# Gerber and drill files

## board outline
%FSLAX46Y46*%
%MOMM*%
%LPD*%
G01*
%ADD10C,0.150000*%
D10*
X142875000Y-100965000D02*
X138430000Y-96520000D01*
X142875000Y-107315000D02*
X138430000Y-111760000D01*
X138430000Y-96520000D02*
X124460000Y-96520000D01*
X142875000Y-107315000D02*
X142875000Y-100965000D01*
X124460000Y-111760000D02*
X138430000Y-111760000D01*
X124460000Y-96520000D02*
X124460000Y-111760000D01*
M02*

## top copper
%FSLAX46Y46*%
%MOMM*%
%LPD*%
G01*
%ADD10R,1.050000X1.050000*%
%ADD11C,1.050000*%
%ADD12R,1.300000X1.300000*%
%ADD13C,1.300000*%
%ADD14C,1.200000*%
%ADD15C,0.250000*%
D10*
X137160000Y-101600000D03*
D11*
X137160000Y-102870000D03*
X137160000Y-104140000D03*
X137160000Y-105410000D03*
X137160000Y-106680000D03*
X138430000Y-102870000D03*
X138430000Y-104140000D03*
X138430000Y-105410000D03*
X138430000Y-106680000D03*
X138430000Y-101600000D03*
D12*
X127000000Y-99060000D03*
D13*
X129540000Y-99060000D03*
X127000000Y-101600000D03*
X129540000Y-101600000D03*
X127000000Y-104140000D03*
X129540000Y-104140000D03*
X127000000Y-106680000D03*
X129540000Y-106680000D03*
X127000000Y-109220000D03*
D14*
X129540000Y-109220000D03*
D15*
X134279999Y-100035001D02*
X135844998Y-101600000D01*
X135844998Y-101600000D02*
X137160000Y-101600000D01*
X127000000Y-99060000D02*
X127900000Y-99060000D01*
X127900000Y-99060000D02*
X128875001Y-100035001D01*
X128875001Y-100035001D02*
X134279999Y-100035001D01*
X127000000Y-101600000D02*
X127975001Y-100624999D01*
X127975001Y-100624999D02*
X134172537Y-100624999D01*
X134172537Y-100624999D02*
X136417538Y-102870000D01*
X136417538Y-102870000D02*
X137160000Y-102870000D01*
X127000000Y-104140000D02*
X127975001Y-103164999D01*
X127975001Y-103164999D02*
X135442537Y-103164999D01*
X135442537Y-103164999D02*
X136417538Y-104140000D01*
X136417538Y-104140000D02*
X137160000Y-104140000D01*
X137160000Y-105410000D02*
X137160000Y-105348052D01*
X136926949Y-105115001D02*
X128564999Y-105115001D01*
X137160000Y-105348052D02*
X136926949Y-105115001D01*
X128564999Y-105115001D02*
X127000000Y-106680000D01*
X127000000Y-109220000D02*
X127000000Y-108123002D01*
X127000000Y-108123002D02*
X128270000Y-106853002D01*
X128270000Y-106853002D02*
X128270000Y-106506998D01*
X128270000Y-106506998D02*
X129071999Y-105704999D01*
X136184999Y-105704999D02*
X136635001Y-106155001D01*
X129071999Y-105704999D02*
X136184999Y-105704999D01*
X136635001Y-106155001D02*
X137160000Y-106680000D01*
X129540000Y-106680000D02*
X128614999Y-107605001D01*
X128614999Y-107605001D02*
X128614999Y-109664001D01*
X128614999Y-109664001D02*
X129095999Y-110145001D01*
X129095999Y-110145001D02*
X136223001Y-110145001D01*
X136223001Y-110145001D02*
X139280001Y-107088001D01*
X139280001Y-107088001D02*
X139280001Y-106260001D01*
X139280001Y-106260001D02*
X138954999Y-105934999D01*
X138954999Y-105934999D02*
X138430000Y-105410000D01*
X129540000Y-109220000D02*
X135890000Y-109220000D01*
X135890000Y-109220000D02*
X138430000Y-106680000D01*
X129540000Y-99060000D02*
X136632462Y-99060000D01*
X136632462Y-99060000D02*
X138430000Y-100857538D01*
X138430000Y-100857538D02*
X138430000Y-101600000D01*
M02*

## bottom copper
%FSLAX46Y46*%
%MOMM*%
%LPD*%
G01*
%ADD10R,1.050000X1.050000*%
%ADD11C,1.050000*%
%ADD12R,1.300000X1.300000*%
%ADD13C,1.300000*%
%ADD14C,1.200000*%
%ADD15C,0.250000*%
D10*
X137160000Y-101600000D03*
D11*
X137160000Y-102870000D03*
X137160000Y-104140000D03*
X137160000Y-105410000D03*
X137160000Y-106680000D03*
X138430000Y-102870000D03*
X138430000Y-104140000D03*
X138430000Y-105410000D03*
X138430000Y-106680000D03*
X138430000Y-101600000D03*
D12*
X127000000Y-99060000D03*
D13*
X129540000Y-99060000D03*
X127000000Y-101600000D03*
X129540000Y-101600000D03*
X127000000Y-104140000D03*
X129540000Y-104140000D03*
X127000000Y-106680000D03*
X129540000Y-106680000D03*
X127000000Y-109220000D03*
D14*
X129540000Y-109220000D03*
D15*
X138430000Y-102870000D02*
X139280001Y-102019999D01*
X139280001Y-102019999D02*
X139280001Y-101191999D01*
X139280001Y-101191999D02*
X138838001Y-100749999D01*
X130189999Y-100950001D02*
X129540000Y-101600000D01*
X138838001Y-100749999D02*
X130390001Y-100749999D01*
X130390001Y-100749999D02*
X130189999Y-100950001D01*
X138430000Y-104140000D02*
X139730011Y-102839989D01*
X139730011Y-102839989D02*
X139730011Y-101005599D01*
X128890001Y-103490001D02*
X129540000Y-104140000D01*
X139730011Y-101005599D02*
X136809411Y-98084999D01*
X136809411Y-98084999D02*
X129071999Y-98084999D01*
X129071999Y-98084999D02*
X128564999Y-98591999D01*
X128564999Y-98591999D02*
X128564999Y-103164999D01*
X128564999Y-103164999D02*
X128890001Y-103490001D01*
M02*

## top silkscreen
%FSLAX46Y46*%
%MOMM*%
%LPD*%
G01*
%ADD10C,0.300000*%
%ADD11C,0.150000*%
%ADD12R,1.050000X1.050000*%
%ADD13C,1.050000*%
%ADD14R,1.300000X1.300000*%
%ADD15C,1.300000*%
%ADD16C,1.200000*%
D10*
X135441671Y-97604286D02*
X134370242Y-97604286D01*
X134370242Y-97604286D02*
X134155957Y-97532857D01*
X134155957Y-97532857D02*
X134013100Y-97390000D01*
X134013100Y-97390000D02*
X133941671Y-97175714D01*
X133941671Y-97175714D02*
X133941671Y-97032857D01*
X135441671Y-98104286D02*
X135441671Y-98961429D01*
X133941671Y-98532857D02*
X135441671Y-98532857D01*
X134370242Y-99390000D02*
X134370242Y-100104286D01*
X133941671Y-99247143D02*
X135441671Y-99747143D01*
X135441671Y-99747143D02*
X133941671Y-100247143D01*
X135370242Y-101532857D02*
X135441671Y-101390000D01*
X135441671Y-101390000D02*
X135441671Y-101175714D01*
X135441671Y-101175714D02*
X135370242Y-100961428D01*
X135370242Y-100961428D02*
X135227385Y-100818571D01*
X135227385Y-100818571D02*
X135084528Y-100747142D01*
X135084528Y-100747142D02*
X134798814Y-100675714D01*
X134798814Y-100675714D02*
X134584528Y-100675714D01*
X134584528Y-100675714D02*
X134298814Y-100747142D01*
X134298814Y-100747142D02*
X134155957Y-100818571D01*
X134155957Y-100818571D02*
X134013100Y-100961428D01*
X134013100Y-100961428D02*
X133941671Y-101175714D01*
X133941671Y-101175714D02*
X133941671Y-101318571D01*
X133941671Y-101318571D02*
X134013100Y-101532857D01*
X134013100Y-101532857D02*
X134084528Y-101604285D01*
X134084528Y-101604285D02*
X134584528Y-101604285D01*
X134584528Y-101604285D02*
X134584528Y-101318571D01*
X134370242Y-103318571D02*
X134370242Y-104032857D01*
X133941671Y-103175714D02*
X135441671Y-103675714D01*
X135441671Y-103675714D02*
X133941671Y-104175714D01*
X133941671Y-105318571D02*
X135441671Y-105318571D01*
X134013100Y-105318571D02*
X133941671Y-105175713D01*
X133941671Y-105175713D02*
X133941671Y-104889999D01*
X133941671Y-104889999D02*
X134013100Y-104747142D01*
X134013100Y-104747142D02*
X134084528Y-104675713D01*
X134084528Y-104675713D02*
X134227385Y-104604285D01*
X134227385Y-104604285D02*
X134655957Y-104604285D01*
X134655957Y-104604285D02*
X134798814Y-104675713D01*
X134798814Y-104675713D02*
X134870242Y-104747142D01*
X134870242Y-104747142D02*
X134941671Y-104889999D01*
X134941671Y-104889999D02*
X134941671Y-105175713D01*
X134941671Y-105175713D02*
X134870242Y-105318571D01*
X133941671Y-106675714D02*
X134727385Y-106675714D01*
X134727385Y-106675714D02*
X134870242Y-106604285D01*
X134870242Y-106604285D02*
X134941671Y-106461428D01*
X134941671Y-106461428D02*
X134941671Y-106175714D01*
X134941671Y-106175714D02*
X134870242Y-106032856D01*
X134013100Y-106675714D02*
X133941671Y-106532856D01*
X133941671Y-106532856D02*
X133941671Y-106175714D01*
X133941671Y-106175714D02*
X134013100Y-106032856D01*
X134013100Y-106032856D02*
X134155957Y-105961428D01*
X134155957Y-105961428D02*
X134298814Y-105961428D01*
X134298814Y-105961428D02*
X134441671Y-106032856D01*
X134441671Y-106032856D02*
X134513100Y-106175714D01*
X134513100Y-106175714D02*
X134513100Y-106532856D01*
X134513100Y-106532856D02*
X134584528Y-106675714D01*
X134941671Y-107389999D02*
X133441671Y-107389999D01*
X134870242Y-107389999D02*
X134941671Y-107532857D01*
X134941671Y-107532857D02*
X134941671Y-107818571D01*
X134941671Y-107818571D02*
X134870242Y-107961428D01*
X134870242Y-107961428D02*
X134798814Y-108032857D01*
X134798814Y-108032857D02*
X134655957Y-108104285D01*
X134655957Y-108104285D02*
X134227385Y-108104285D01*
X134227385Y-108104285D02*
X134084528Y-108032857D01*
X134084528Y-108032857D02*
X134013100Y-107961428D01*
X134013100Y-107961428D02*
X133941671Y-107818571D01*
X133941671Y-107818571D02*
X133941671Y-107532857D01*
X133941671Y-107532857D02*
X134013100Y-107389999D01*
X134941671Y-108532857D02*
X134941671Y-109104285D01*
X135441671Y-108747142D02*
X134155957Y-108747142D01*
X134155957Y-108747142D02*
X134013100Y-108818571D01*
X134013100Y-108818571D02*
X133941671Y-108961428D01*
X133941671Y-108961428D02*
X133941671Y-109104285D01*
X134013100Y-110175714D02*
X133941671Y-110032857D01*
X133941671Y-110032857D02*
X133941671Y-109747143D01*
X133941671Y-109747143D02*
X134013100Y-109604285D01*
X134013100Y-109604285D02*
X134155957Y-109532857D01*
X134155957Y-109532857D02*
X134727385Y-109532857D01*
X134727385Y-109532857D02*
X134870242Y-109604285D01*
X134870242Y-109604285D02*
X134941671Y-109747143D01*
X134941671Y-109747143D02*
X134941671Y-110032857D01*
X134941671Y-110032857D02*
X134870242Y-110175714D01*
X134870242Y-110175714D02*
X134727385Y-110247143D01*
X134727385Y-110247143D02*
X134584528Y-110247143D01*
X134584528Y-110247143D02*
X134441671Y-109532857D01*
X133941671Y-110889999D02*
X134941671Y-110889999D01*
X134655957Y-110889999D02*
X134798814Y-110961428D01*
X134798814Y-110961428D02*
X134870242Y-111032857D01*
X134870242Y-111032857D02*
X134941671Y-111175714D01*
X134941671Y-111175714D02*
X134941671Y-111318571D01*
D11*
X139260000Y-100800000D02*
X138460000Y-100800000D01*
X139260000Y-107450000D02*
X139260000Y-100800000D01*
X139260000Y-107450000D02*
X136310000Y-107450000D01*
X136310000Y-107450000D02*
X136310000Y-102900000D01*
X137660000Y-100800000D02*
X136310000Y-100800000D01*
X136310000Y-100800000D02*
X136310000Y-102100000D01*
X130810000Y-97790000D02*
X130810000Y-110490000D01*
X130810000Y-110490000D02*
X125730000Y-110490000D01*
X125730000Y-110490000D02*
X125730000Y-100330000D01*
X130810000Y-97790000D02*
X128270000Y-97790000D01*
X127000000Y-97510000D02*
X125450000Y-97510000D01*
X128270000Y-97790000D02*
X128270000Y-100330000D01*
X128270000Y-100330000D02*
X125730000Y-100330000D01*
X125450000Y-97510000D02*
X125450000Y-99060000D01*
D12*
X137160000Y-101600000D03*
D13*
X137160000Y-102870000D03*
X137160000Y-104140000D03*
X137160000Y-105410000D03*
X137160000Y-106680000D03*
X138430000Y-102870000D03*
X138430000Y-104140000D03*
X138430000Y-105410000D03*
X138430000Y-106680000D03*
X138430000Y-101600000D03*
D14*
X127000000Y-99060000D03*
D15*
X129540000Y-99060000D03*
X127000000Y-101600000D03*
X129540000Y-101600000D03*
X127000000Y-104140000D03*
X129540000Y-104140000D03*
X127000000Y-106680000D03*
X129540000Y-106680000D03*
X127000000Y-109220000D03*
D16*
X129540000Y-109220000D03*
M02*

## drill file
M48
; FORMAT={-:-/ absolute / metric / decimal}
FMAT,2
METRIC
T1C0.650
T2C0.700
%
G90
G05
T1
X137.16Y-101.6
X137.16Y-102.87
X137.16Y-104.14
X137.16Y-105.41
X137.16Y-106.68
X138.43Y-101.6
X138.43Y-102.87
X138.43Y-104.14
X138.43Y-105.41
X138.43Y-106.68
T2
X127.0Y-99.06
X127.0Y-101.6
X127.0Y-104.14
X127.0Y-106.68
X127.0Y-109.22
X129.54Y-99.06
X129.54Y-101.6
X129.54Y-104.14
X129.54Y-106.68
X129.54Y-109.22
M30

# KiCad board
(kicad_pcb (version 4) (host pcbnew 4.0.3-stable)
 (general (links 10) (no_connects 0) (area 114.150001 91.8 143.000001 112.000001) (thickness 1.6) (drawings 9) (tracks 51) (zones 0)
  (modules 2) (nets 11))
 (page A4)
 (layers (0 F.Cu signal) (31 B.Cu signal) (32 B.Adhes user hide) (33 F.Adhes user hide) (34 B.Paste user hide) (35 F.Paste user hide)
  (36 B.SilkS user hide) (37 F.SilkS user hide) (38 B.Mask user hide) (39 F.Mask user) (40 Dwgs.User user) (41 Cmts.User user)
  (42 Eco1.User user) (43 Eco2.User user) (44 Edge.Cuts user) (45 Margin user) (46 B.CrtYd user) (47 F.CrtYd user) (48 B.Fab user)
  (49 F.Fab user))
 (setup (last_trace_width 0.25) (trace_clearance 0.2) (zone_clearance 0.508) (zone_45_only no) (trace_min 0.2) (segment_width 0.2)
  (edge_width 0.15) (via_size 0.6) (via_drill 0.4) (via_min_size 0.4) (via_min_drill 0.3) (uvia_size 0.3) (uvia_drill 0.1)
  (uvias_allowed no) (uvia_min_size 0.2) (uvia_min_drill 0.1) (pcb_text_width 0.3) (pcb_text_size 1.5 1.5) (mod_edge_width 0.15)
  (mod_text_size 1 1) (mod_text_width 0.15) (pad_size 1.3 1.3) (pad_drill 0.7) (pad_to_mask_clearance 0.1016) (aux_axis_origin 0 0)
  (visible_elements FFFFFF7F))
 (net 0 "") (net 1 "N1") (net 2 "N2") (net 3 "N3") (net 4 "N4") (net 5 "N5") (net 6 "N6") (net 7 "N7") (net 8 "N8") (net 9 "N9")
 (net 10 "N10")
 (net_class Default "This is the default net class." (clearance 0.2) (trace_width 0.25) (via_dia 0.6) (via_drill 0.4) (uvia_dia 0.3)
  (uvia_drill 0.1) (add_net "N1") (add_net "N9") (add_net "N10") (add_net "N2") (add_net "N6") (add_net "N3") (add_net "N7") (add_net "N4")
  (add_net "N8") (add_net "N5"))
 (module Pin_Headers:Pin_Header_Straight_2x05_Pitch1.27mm (layer F.Cu) (at 137.16 101.6)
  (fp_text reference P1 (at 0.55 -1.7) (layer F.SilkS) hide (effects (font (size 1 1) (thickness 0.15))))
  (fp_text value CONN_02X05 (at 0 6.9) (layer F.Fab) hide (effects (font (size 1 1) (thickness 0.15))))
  (fp_line (start 2.1 -0.8) (end 1.3 -0.8) (layer F.SilkS) (width 0.15))
  (fp_line (start 2.1 5.85) (end 2.1 -0.8) (layer F.SilkS) (width 0.15))
  (fp_line (start 2.1 5.85) (end -0.85 5.85) (layer F.SilkS) (width 0.15))
  (fp_line (start -0.85 5.85) (end -0.85 1.3) (layer F.SilkS) (width 0.15))
  (fp_line (start 0.5 -0.8) (end -0.85 -0.8) (layer F.SilkS) (width 0.15))
  (fp_line (start -0.85 -0.8) (end -0.85 0.5) (layer F.SilkS) (width 0.15))
  (pad 1 thru_hole rect (at 0 0) (size 1.05 1.05) (drill 0.65) (layers *.Cu *.Mask F.SilkS) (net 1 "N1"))
  (pad 3 thru_hole circle (at 0 1.27) (size 1.05 1.05) (drill 0.65) (layers *.Cu *.Mask F.SilkS) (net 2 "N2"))
  (pad 5 thru_hole circle (at 0 2.54) (size 1.05 1.05) (drill 0.65) (layers *.Cu *.Mask F.SilkS) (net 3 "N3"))
  (pad 7 thru_hole circle (at 0 3.81) (size 1.05 1.05) (drill 0.65) (layers *.Cu *.Mask F.SilkS) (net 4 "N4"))
  (pad 9 thru_hole circle (at 0 5.08) (size 1.05 1.05) (drill 0.65) (layers *.Cu *.Mask F.SilkS) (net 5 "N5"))
  (pad 4 thru_hole circle (at 1.27 1.27) (size 1.05 1.05) (drill 0.65) (layers *.Cu *.Mask F.SilkS) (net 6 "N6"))
  (pad 6 thru_hole circle (at 1.27 2.54) (size 1.05 1.05) (drill 0.65) (layers *.Cu *.Mask F.SilkS) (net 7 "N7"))
  (pad 8 thru_hole circle (at 1.27 3.81) (size 1.05 1.05) (drill 0.65) (layers *.Cu *.Mask F.SilkS) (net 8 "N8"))
  (pad 10 thru_hole circle (at 1.27 5.08) (size 1.05 1.05) (drill 0.65) (layers *.Cu *.Mask F.SilkS) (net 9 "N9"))
  (pad 2 thru_hole circle (at 1.27 0) (size 1.05 1.05) (drill 0.65) (layers *.Cu *.Mask F.SilkS) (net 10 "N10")))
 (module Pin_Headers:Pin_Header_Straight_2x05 (layer F.Cu) (at 127 99.06)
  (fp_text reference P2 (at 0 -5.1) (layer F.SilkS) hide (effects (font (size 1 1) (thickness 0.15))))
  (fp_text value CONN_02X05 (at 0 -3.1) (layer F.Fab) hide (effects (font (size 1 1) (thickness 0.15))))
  (fp_line (start 3.81 -1.27) (end 3.81 11.43) (layer F.SilkS) (width 0.15))
  (fp_line (start 3.81 11.43) (end -1.27 11.43) (layer F.SilkS) (width 0.15))
  (fp_line (start -1.27 11.43) (end -1.27 1.27) (layer F.SilkS) (width 0.15))
  (fp_line (start 3.81 -1.27) (end 1.27 -1.27) (layer F.SilkS) (width 0.15))
  (fp_line (start 0 -1.55) (end -1.55 -1.55) (layer F.SilkS) (width 0.15))
  (fp_line (start 1.27 -1.27) (end 1.27 1.27) (layer F.SilkS) (width 0.15))
  (fp_line (start 1.27 1.27) (end -1.27 1.27) (layer F.SilkS) (width 0.15))
  (fp_line (start -1.55 -1.55) (end -1.55 0) (layer F.SilkS) (width 0.15))
  (pad 1 thru_hole rect (at 0 0) (size 1.3 1.3) (drill 0.7) (layers *.Cu *.Mask F.SilkS) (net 1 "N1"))
  (pad 2 thru_hole circle (at 2.54 0) (size 1.3 1.3) (drill 0.7) (layers *.Cu *.Mask F.SilkS) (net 10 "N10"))
  (pad 3 thru_hole circle (at 0 2.54) (size 1.3 1.3) (drill 0.7) (layers *.Cu *.Mask F.SilkS) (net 2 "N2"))
  (pad 4 thru_hole circle (at 2.54 2.54) (size 1.3 1.3) (drill 0.7) (layers *.Cu *.Mask F.SilkS) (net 6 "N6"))
  (pad 5 thru_hole circle (at 0 5.08) (size 1.3 1.3) (drill 0.7) (layers *.Cu *.Mask F.SilkS) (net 3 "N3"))
  (pad 6 thru_hole circle (at 2.54 5.08) (size 1.3 1.3) (drill 0.7) (layers *.Cu *.Mask F.SilkS) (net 7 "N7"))
  (pad 7 thru_hole circle (at 0 7.62) (size 1.3 1.3) (drill 0.7) (layers *.Cu *.Mask F.SilkS) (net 4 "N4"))
  (pad 8 thru_hole circle (at 2.54 7.62) (size 1.3 1.3) (drill 0.7) (layers *.Cu *.Mask F.SilkS) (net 8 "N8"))
  (pad 9 thru_hole circle (at 0 10.16) (size 1.3 1.3) (drill 0.7) (layers *.Cu *.Mask F.SilkS) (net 5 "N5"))
  (pad 10 thru_hole circle (at 2.54 10.16) (size 1.2 1.2) (drill 0.7) (layers *.Cu *.Mask F.SilkS) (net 9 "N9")))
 (gr_line (start 142.875 100.965) (end 138.43 96.52) (layer Edge.Cuts) (width 0.15))
 (gr_line (start 142.875 107.315) (end 138.43 111.76) (layer Edge.Cuts) (width 0.15))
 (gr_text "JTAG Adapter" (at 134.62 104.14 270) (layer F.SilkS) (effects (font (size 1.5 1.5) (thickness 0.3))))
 (gr_line (start 138.43 96.52) (end 124.46 96.52) (layer Edge.Cuts) (width 0.15))
 (gr_line (start 142.875 107.315) (end 142.875 100.965) (layer Edge.Cuts) (width 0.15))
 (gr_line (start 124.46 111.76) (end 138.43 111.76) (layer Edge.Cuts) (width 0.15))
 (gr_line (start 124.46 96.52) (end 124.46 111.76) (layer Edge.Cuts) (width 0.15))
 (segment (start 134.279999 100.035001) (end 135.844998 101.6) (width 0.25) (layer F.Cu) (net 1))
 (segment (start 135.844998 101.6) (end 137.16 101.6) (width 0.25) (layer F.Cu) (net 1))
 (segment (start 127 99.06) (end 127.9 99.06) (width 0.25) (layer F.Cu) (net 1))
 (segment (start 127.9 99.06) (end 128.875001 100.035001) (width 0.25) (layer F.Cu) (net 1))
 (segment (start 128.875001 100.035001) (end 134.279999 100.035001) (width 0.25) (layer F.Cu) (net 1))
 (segment (start 127 101.6) (end 127.975001 100.624999) (width 0.25) (layer F.Cu) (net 2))
 (segment (start 127.975001 100.624999) (end 134.172537 100.624999) (width 0.25) (layer F.Cu) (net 2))
 (segment (start 134.172537 100.624999) (end 136.417538 102.87) (width 0.25) (layer F.Cu) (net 2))
 (segment (start 136.417538 102.87) (end 137.16 102.87) (width 0.25) (layer F.Cu) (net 2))
 (segment (start 127 104.14) (end 127.975001 103.164999) (width 0.25) (layer F.Cu) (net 3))
 (segment (start 127.975001 103.164999) (end 135.442537 103.164999) (width 0.25) (layer F.Cu) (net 3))
 (segment (start 135.442537 103.164999) (end 136.417538 104.14) (width 0.25) (layer F.Cu) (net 3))
 (segment (start 136.417538 104.14) (end 137.16 104.14) (width 0.25) (layer F.Cu) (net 3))
 (segment (start 137.16 105.41) (end 137.16 105.348052) (width 0.25) (layer F.Cu) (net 4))
 (segment (start 136.926949 105.115001) (end 128.564999 105.115001) (width 0.25) (layer F.Cu) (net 4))
 (segment (start 137.16 105.348052) (end 136.926949 105.115001) (width 0.25) (layer F.Cu) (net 4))
 (segment (start 128.564999 105.115001) (end 127 106.68) (width 0.25) (layer F.Cu) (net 4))
 (segment (start 127 109.22) (end 127 108.123002) (width 0.25) (layer F.Cu) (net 5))
 (segment (start 127 108.123002) (end 128.27 106.853002) (width 0.25) (layer F.Cu) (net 5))
 (segment (start 128.27 106.853002) (end 128.27 106.506998) (width 0.25) (layer F.Cu) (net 5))
 (segment (start 128.27 106.506998) (end 129.071999 105.704999) (width 0.25) (layer F.Cu) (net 5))
 (segment (start 136.184999 105.704999) (end 136.635001 106.155001) (width 0.25) (layer F.Cu) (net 5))
 (segment (start 129.071999 105.704999) (end 136.184999 105.704999) (width 0.25) (layer F.Cu) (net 5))
 (segment (start 136.635001 106.155001) (end 137.16 106.68) (width 0.25) (layer F.Cu) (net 5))
 (segment (start 138.43 102.87) (end 139.280001 102.019999) (width 0.25) (layer B.Cu) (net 6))
 (segment (start 139.280001 102.019999) (end 139.280001 101.191999) (width 0.25) (layer B.Cu) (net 6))
 (segment (start 139.280001 101.191999) (end 138.838001 100.749999) (width 0.25) (layer B.Cu) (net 6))
 (segment (start 130.189999 100.950001) (end 129.54 101.6) (width 0.25) (layer B.Cu) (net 6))
 (segment (start 138.838001 100.749999) (end 130.390001 100.749999) (width 0.25) (layer B.Cu) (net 6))
 (segment (start 130.390001 100.749999) (end 130.189999 100.950001) (width 0.25) (layer B.Cu) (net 6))
 (segment (start 138.43 104.14) (end 139.730011 102.839989) (width 0.25) (layer B.Cu) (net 7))
 (segment (start 139.730011 102.839989) (end 139.730011 101.005599) (width 0.25) (layer B.Cu) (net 7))
 (segment (start 128.890001 103.490001) (end 129.54 104.14) (width 0.25) (layer B.Cu) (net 7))
 (segment (start 139.730011 101.005599) (end 136.809411 98.084999) (width 0.25) (layer B.Cu) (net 7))
 (segment (start 136.809411 98.084999) (end 129.071999 98.084999) (width 0.25) (layer B.Cu) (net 7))
 (segment (start 129.071999 98.084999) (end 128.564999 98.591999) (width 0.25) (layer B.Cu) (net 7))
 (segment (start 128.564999 98.591999) (end 128.564999 103.164999) (width 0.25) (layer B.Cu) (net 7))
 (segment (start 128.564999 103.164999) (end 128.890001 103.490001) (width 0.25) (layer B.Cu) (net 7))
 (segment (start 129.54 106.68) (end 128.614999 107.605001) (width 0.25) (layer F.Cu) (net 8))
 (segment (start 128.614999 107.605001) (end 128.614999 109.664001) (width 0.25) (layer F.Cu) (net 8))
 (segment (start 128.614999 109.664001) (end 129.095999 110.145001) (width 0.25) (layer F.Cu) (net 8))
 (segment (start 129.095999 110.145001) (end 136.223001 110.145001) (width 0.25) (layer F.Cu) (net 8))
 (segment (start 136.223001 110.145001) (end 139.280001 107.088001) (width 0.25) (layer F.Cu) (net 8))
 (segment (start 139.280001 107.088001) (end 139.280001 106.260001) (width 0.25) (layer F.Cu) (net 8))
 (segment (start 139.280001 106.260001) (end 138.954999 105.934999) (width 0.25) (layer F.Cu) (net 8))
 (segment (start 138.954999 105.934999) (end 138.43 105.41) (width 0.25) (layer F.Cu) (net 8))
 (segment (start 129.54 109.22) (end 135.89 109.22) (width 0.25) (layer F.Cu) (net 9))
 (segment (start 135.89 109.22) (end 138.43 106.68) (width 0.25) (layer F.Cu) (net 9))
 (segment (start 129.54 99.06) (end 136.632462 99.06) (width 0.25) (layer F.Cu) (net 10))
 (segment (start 136.632462 99.06) (end 138.43 100.857538) (width 0.25) (layer F.Cu) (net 10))
 (segment (start 138.43 100.857538) (end 138.43 101.6) (width 0.25) (layer F.Cu) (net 10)))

